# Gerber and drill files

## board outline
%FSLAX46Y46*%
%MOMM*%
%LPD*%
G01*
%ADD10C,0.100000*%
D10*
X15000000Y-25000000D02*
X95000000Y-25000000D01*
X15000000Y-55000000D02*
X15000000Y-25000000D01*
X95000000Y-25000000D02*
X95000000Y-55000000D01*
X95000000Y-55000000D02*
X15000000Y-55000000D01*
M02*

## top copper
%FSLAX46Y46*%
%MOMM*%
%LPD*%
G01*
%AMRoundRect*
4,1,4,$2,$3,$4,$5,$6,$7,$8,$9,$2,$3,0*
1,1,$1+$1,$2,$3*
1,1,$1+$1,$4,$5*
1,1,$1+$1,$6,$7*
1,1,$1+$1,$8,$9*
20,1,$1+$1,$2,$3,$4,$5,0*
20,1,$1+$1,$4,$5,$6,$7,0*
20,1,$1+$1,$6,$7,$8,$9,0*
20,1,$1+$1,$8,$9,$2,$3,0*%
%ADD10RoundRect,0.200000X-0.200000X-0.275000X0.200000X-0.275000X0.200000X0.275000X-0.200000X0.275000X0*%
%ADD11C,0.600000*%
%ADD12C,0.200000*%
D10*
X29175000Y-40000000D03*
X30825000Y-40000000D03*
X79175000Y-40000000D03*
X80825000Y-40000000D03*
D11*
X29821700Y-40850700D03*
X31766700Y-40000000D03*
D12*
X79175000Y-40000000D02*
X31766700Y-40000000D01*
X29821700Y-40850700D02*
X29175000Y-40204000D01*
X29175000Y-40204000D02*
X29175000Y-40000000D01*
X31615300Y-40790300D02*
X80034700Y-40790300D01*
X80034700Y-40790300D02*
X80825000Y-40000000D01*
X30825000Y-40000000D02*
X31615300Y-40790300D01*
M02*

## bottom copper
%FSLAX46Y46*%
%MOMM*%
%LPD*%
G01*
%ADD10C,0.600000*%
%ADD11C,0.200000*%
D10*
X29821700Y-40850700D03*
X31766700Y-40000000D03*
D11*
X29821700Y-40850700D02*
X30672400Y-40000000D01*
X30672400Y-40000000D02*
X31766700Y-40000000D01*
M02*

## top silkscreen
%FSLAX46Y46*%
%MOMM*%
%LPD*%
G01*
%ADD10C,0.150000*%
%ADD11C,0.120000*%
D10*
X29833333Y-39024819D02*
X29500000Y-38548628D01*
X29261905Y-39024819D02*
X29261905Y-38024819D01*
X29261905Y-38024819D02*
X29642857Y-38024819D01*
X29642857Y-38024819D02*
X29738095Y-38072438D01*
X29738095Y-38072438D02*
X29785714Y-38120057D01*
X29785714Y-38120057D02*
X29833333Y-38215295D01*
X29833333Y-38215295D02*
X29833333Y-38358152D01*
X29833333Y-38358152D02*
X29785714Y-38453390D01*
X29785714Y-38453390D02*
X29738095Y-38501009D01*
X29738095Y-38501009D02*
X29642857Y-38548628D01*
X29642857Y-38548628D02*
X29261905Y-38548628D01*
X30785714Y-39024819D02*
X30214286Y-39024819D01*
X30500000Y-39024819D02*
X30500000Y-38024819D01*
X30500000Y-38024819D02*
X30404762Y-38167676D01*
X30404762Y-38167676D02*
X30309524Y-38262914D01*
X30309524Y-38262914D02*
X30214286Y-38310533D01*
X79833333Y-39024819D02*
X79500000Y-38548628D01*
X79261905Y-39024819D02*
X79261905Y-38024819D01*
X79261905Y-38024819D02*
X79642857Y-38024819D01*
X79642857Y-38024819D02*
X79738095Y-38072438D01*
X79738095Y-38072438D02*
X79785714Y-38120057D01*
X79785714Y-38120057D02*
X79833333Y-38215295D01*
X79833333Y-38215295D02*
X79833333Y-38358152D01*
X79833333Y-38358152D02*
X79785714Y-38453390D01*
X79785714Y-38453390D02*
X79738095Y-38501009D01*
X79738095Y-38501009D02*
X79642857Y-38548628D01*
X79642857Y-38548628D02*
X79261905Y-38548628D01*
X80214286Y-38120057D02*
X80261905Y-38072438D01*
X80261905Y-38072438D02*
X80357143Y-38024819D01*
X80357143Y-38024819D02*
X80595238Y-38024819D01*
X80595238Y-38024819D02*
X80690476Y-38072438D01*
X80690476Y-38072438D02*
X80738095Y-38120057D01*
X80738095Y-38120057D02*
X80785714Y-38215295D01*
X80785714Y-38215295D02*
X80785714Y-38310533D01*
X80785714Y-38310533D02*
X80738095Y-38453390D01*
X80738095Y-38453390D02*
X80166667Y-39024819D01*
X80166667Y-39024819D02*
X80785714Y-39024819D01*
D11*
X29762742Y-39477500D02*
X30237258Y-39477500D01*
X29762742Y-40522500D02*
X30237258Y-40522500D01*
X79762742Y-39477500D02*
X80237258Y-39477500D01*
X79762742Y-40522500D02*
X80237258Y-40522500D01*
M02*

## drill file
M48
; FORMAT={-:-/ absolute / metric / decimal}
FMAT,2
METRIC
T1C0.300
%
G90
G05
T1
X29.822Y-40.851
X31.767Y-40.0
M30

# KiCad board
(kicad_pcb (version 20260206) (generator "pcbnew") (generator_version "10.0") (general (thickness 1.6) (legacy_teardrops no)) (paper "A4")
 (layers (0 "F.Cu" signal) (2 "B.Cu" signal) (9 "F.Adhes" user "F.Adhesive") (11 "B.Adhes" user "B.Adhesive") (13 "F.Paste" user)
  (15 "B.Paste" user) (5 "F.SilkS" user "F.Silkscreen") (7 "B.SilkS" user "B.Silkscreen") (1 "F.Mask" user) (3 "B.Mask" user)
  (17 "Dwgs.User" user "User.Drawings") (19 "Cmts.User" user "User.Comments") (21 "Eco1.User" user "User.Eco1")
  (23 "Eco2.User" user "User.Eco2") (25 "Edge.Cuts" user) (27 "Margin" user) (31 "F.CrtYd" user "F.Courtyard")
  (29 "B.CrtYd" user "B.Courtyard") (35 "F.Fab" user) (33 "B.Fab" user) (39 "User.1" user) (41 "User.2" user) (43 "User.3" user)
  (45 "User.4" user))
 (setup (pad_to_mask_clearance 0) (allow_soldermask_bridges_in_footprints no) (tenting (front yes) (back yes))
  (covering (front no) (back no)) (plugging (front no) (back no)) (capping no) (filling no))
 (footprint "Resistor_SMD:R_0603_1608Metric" (layer "F.Cu") (at 30 40)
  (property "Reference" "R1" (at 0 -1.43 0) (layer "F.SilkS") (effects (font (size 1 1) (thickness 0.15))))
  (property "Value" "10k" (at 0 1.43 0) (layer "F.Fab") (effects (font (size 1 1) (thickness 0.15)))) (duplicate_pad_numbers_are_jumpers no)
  (fp_line (start -0.237258 -0.5225) (end 0.237258 -0.5225) (stroke (width 0.12) (type solid)) (layer "F.SilkS"))
  (fp_line (start -0.237258 0.5225) (end 0.237258 0.5225) (stroke (width 0.12) (type solid)) (layer "F.SilkS"))
  (pad "1" smd roundrect (at -0.825 0) (size 0.8 0.95) (layers "F.Cu" "F.Mask" "F.Paste") (roundrect_rratio 0.25) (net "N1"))
  (pad "2" smd roundrect (at 0.825 0) (size 0.8 0.95) (layers "F.Cu" "F.Mask" "F.Paste") (roundrect_rratio 0.25) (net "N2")))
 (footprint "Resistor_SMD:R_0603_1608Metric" (layer "F.Cu") (at 80 40)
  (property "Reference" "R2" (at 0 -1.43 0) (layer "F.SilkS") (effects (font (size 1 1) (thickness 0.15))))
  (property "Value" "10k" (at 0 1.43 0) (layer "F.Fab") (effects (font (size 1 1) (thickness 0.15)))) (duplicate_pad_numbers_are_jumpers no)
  (fp_line (start -0.237258 -0.5225) (end 0.237258 -0.5225) (stroke (width 0.12) (type solid)) (layer "F.SilkS"))
  (fp_line (start -0.237258 0.5225) (end 0.237258 0.5225) (stroke (width 0.12) (type solid)) (layer "F.SilkS"))
  (pad "1" smd roundrect (at -0.825 0) (size 0.8 0.95) (layers "F.Cu" "F.Mask" "F.Paste") (roundrect_rratio 0.25) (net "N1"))
  (pad "2" smd roundrect (at 0.825 0) (size 0.8 0.95) (layers "F.Cu" "F.Mask" "F.Paste") (roundrect_rratio 0.25) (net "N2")))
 (gr_line (start 15 25) (end 95 25) (stroke (width 0.1) (type default)) (layer "Edge.Cuts"))
 (gr_line (start 15 55) (end 15 25) (stroke (width 0.1) (type default)) (layer "Edge.Cuts"))
 (gr_line (start 95 25) (end 95 55) (stroke (width 0.1) (type default)) (layer "Edge.Cuts"))
 (gr_line (start 95 55) (end 15 55) (stroke (width 0.1) (type default)) (layer "Edge.Cuts"))
 (segment (start 79.175 40) (end 31.7667 40) (width 0.2) (layer "F.Cu") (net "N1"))
 (segment (start 29.8217 40.8507) (end 29.175 40.204) (width 0.2) (layer "F.Cu") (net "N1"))
 (segment (start 29.175 40.204) (end 29.175 40) (width 0.2) (layer "F.Cu") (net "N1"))
 (via (at 29.8217 40.8507) (size 0.6) (drill 0.3) (layers "F.Cu" "B.Cu") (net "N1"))
 (via (at 31.7667 40) (size 0.6) (drill 0.3) (layers "F.Cu" "B.Cu") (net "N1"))
 (segment (start 29.8217 40.8507) (end 30.6724 40) (width 0.2) (layer "B.Cu") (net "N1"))
 (segment (start 30.6724 40) (end 31.7667 40) (width 0.2) (layer "B.Cu") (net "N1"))
 (segment (start 31.6153 40.7903) (end 80.0347 40.7903) (width 0.2) (layer "F.Cu") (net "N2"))
 (segment (start 80.0347 40.7903) (end 80.825 40) (width 0.2) (layer "F.Cu") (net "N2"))
 (segment (start 30.825 40) (end 31.6153 40.7903) (width 0.2) (layer "F.Cu") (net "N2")))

